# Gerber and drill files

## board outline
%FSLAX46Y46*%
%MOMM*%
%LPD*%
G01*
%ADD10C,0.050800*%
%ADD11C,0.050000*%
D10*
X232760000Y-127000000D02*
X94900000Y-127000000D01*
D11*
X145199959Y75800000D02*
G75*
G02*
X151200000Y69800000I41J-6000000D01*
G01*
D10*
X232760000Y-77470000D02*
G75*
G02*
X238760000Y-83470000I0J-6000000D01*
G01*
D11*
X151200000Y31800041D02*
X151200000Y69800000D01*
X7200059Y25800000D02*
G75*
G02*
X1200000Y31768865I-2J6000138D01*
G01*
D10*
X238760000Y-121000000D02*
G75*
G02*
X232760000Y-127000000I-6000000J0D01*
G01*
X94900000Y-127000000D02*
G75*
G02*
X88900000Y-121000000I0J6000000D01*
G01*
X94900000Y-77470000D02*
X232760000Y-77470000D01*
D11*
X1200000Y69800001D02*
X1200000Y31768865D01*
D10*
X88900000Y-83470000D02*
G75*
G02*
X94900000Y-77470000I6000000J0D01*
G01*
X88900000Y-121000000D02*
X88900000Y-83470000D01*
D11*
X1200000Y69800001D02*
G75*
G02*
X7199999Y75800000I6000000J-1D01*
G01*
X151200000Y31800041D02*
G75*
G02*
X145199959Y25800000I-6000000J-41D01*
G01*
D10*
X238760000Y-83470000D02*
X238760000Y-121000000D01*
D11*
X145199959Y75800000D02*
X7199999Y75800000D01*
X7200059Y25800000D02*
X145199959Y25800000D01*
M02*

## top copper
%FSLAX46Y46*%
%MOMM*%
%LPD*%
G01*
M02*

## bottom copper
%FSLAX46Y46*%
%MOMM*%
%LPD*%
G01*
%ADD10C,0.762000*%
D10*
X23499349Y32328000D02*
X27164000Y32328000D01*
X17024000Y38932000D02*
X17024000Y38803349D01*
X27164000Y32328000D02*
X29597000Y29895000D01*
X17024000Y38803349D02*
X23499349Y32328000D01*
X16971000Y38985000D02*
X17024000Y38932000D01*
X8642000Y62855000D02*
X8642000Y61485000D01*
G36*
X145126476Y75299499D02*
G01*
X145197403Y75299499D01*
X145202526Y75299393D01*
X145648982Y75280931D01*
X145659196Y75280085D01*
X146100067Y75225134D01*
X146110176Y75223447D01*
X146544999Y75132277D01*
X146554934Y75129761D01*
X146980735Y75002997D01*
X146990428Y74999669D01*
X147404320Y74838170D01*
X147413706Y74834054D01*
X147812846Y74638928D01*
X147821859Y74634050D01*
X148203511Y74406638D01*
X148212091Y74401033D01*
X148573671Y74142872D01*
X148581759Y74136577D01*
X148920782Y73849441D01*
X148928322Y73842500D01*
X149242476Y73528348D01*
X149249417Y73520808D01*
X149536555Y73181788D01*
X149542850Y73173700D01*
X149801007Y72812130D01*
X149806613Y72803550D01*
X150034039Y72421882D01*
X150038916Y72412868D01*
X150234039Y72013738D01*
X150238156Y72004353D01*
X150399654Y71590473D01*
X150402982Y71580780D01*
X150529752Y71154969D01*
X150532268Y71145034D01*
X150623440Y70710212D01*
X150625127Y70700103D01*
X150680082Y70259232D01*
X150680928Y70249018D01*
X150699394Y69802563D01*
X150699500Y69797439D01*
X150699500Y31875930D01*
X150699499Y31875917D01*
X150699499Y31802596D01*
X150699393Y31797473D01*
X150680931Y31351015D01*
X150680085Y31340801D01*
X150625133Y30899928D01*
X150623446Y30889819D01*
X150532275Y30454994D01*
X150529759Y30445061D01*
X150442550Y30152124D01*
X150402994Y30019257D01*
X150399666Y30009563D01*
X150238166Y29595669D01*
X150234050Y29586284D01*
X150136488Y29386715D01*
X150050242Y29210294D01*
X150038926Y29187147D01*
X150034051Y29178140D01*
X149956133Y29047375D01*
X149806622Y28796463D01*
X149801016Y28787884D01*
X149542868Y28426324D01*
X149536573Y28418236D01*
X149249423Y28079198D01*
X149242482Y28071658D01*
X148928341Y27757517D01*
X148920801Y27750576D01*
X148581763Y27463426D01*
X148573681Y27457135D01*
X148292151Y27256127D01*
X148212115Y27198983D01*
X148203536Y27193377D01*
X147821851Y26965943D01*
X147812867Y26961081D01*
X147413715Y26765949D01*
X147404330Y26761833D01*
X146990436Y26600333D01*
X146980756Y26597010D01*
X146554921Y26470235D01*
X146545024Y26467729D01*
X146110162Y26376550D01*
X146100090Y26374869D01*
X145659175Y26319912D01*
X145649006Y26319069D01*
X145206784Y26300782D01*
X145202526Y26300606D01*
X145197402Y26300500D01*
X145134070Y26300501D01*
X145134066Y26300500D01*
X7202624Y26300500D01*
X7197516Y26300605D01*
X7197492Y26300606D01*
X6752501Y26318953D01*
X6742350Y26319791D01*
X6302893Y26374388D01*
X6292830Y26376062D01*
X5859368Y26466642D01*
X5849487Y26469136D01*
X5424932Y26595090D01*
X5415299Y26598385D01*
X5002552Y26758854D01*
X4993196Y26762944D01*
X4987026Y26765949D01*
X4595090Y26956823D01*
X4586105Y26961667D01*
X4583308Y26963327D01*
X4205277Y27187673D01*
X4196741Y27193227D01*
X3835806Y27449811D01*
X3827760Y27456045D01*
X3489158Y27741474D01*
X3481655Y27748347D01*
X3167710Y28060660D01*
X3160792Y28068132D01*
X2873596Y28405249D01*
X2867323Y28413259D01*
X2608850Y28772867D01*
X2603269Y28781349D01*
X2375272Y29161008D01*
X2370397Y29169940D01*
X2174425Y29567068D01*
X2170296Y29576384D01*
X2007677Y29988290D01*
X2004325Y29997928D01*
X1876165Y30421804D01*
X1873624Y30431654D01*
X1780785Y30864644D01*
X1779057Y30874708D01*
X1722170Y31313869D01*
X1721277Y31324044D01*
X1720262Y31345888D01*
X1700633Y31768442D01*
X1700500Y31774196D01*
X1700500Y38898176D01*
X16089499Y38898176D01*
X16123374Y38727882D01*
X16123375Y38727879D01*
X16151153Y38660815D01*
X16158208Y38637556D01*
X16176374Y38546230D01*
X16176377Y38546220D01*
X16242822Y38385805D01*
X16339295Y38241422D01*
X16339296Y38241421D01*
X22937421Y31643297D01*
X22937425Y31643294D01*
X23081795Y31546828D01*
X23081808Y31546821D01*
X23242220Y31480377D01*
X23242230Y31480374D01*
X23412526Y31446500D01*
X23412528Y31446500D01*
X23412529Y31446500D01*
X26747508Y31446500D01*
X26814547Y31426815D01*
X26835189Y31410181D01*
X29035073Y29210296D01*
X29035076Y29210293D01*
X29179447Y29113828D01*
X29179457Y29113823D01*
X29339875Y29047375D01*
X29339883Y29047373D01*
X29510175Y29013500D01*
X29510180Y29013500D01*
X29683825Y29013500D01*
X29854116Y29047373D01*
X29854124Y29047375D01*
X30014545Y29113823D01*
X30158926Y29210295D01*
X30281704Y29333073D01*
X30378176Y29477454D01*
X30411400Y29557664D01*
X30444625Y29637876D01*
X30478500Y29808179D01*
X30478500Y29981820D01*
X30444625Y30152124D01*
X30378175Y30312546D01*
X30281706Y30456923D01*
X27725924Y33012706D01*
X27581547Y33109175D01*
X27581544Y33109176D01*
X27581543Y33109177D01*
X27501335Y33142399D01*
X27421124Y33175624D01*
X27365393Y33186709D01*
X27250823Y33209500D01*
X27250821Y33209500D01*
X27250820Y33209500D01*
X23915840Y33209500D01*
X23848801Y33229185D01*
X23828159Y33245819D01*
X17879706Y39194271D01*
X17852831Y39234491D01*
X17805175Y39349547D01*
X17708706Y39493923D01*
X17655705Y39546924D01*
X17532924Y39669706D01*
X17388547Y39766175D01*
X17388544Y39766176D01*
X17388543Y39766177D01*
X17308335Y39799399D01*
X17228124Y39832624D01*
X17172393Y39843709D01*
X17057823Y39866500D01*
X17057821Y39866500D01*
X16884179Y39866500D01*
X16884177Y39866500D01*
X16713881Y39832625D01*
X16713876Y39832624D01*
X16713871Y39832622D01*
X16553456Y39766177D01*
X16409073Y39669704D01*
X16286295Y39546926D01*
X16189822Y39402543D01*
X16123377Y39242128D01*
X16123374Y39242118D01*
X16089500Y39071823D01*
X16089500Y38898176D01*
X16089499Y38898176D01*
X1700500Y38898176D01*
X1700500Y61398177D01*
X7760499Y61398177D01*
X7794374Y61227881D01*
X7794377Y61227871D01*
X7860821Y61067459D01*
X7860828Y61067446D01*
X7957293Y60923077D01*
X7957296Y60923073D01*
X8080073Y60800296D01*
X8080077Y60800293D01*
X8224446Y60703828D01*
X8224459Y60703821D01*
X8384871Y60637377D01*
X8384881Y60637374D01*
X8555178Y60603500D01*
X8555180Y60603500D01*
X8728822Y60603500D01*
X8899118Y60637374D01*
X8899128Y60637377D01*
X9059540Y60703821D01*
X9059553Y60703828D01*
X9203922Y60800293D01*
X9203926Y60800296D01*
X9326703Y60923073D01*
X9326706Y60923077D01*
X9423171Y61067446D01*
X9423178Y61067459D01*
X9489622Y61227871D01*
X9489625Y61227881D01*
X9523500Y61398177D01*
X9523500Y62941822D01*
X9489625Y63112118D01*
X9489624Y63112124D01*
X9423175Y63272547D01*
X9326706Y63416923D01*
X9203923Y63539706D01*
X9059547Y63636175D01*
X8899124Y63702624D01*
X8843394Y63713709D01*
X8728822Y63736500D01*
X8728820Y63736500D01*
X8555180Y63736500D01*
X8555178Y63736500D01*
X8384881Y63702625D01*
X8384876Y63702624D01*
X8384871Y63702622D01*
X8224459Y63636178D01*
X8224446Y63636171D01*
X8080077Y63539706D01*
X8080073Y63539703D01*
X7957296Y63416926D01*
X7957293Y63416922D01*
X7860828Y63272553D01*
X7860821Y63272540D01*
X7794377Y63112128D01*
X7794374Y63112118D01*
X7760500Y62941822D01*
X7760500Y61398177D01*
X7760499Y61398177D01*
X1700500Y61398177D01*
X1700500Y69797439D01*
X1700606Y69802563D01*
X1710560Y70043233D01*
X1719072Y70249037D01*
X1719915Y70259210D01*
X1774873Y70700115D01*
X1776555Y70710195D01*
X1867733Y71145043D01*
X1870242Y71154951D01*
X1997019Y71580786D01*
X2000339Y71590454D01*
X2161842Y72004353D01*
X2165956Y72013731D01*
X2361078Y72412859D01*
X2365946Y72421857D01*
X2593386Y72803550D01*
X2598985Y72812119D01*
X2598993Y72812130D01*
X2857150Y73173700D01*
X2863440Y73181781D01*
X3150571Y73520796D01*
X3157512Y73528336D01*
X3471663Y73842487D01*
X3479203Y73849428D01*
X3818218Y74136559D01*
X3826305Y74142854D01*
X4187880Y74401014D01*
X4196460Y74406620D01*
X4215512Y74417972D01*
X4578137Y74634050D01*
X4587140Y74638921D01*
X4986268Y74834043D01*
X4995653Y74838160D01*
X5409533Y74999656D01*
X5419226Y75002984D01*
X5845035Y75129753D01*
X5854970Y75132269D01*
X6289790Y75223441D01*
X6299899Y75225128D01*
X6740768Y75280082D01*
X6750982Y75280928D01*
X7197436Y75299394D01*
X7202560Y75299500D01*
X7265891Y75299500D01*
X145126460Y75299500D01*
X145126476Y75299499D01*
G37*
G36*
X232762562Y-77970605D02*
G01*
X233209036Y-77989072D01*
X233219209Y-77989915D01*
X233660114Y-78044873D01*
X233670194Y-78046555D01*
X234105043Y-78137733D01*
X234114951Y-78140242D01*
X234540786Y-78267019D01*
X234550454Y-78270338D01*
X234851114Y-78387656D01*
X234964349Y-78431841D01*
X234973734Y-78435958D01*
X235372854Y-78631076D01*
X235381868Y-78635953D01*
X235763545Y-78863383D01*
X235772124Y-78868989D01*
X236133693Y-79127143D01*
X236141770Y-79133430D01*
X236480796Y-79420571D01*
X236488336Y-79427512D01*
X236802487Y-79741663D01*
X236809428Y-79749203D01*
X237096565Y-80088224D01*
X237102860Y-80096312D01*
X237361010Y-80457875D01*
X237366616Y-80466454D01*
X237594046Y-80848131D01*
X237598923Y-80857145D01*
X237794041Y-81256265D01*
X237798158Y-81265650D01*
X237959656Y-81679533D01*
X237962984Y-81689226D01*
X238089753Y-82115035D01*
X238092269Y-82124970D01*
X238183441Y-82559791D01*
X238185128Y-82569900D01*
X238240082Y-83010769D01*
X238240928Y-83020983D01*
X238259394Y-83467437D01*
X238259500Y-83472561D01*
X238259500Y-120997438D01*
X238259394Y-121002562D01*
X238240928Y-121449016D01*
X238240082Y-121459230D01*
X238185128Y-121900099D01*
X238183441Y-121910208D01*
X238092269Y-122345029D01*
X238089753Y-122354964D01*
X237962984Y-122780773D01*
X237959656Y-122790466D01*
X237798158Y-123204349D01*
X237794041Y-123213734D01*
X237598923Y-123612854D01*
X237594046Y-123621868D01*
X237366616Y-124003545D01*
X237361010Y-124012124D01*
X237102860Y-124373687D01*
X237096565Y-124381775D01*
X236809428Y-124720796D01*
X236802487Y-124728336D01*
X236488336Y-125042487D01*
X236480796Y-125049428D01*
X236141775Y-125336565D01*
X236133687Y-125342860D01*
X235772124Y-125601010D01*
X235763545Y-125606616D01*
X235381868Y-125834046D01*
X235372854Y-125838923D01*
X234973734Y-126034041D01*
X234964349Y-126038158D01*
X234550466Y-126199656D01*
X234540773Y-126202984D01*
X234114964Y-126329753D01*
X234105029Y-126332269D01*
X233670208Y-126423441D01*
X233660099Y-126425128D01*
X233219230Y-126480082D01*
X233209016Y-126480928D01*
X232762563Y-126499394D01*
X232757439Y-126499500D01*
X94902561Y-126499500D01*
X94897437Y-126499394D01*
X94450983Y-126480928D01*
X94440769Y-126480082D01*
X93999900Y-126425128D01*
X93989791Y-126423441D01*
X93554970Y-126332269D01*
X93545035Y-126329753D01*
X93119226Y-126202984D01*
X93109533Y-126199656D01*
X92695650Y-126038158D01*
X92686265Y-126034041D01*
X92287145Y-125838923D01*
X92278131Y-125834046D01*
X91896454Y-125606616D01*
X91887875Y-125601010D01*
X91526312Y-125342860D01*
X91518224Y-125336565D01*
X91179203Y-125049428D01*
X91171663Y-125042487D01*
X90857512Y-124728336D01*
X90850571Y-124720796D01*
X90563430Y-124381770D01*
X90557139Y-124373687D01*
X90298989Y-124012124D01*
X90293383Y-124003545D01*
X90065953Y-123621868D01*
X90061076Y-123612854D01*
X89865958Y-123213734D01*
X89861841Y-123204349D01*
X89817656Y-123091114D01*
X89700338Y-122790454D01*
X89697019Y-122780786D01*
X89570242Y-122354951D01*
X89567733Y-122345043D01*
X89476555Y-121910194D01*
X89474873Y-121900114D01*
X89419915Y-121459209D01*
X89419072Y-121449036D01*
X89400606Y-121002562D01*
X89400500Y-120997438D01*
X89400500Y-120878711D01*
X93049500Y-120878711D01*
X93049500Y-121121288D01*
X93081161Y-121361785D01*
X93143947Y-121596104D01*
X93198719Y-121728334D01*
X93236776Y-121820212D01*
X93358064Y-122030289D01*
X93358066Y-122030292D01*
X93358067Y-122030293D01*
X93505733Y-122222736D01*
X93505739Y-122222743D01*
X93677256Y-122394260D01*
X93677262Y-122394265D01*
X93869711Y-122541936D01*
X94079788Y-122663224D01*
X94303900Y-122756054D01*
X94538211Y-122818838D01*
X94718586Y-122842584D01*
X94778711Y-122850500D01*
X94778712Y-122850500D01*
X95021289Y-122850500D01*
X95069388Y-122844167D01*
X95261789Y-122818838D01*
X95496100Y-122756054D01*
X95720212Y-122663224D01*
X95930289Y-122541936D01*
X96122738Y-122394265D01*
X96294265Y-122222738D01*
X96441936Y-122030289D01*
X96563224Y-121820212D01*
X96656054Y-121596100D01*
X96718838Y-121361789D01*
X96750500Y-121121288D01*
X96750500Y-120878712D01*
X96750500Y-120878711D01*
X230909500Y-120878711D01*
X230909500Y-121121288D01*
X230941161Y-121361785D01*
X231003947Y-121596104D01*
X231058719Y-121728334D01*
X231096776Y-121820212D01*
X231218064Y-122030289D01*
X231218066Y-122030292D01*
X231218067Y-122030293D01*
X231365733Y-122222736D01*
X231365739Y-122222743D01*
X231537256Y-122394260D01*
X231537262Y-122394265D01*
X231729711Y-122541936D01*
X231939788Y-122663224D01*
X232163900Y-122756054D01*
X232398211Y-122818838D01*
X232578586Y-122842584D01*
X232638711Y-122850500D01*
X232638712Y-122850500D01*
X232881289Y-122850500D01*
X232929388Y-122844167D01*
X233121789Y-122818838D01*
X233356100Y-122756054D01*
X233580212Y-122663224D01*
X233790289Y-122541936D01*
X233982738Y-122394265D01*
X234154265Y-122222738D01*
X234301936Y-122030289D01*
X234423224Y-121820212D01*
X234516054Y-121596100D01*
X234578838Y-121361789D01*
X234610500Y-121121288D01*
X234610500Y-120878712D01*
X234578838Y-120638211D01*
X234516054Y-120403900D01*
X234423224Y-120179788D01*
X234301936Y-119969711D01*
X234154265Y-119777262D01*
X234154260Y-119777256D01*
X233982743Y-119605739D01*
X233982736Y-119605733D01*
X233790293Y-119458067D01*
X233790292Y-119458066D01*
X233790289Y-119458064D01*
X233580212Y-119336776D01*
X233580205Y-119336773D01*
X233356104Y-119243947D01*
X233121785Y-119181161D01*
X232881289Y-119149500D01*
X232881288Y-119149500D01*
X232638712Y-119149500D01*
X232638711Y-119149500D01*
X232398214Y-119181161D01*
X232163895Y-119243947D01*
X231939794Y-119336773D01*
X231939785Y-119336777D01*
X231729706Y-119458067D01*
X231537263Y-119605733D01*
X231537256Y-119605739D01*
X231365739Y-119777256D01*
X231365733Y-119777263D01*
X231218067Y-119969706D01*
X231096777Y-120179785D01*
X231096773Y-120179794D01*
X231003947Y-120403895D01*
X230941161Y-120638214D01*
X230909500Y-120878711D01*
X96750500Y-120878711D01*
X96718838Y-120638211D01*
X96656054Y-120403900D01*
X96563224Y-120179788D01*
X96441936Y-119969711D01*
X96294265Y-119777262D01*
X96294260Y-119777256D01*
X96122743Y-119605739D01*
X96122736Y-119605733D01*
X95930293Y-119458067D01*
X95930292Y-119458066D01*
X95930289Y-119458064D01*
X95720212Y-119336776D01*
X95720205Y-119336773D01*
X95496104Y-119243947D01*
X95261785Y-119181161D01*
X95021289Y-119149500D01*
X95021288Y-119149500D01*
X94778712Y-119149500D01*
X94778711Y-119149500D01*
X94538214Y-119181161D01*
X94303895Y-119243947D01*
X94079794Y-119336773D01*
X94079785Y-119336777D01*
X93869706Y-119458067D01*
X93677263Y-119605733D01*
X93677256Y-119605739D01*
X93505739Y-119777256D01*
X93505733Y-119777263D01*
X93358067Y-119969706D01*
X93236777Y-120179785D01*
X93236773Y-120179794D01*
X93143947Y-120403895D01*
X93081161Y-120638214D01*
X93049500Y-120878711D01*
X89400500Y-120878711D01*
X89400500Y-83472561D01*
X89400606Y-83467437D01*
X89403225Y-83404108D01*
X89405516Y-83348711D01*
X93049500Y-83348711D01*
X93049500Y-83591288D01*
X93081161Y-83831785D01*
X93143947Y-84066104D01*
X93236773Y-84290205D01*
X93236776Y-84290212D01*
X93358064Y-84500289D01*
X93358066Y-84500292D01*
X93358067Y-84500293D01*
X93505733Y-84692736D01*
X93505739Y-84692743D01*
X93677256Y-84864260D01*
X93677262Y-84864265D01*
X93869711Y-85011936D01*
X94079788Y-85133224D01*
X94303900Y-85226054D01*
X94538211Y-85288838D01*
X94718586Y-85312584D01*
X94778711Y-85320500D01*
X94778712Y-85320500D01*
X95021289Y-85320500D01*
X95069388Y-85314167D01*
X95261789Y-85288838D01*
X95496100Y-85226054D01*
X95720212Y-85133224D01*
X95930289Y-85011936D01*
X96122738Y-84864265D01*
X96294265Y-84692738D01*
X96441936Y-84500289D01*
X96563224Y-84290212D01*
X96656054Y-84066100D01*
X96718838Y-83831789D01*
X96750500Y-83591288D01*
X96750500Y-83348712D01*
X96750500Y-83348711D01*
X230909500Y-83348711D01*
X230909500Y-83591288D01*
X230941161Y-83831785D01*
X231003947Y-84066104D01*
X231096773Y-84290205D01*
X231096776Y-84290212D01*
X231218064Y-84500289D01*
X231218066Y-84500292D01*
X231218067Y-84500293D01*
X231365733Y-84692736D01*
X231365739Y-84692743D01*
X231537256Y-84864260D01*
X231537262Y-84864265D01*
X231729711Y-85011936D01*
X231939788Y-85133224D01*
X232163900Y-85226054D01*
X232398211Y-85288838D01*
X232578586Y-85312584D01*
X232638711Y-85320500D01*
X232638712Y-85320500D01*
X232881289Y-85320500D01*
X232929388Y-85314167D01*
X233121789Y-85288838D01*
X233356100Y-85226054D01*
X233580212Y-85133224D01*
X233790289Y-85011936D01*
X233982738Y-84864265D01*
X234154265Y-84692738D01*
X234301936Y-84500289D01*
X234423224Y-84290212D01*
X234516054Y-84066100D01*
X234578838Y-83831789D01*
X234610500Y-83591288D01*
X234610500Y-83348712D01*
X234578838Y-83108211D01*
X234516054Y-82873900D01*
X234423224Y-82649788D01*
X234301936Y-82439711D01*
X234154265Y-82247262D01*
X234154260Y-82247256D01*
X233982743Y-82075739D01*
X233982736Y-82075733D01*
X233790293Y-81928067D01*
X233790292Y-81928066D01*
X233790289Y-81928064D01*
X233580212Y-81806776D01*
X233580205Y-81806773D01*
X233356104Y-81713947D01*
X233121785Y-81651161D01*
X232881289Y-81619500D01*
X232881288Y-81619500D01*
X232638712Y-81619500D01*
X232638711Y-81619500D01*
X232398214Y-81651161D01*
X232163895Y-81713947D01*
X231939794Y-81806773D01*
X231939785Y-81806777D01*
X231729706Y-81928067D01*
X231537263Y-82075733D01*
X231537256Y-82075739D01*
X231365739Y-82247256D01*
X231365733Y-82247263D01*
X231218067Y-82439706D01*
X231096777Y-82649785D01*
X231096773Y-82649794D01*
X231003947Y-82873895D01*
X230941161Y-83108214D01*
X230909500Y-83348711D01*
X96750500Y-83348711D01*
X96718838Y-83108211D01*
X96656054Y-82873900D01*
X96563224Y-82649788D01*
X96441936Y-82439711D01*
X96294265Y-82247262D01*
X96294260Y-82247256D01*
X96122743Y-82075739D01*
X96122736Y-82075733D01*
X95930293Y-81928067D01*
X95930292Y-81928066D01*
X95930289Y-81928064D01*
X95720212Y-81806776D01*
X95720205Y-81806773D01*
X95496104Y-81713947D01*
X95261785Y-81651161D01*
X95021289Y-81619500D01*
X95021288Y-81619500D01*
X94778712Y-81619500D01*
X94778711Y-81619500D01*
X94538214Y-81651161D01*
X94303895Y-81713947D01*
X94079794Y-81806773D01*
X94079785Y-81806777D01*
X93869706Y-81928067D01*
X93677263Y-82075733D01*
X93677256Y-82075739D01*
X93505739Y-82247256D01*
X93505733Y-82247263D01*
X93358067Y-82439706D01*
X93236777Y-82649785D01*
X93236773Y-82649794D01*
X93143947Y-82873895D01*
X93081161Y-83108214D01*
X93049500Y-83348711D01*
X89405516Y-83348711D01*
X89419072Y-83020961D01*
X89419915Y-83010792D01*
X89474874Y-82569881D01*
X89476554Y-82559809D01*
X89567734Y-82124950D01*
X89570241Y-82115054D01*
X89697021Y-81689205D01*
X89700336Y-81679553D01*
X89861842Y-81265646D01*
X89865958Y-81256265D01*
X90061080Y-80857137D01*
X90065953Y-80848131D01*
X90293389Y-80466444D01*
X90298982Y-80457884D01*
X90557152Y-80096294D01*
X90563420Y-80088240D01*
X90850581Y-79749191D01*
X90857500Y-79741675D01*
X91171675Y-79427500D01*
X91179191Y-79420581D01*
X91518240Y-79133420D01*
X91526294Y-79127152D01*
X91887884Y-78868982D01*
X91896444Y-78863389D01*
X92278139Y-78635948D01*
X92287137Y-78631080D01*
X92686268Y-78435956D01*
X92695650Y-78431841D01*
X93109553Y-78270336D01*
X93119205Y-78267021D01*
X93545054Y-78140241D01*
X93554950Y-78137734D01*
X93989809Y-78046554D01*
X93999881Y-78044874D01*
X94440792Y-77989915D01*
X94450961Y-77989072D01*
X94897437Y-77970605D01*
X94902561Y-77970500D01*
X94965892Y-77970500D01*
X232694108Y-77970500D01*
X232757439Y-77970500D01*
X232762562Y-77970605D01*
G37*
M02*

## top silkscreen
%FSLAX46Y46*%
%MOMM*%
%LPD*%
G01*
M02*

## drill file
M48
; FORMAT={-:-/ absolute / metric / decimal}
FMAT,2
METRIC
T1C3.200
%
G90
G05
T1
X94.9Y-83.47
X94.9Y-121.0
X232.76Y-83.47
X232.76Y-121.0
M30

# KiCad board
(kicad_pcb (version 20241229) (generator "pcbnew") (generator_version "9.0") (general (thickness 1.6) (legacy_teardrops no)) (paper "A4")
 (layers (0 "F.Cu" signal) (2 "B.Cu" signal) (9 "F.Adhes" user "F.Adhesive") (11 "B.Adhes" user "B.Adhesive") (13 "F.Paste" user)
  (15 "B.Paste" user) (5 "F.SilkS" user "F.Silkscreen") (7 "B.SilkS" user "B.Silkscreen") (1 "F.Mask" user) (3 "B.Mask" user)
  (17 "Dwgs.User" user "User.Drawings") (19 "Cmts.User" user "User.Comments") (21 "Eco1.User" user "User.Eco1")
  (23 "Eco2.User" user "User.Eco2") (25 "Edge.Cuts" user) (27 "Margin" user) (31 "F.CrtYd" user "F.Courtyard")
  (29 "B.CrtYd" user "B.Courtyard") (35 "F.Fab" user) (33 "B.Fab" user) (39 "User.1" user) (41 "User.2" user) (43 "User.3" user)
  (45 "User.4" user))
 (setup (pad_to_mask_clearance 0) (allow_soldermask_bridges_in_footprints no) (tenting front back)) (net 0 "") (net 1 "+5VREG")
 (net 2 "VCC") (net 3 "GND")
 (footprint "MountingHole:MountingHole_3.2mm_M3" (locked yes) (layer "F.Cu") (at 232.76 121)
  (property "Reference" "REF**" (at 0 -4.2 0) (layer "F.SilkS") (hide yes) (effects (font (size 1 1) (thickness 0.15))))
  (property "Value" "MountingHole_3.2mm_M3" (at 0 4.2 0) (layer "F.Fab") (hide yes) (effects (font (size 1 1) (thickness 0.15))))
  (pad "" np_thru_hole circle (at 0 0) (size 3.2 3.2) (drill 3.2) (layers "*.Cu" "*.Mask")))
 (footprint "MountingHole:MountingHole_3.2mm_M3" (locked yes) (layer "F.Cu") (at 94.9 83.47)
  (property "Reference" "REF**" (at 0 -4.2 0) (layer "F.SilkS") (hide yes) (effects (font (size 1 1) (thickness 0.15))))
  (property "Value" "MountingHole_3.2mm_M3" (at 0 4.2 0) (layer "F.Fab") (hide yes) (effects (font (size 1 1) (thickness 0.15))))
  (pad "" np_thru_hole circle (at 0 0) (size 3.2 3.2) (drill 3.2) (layers "*.Cu" "*.Mask")))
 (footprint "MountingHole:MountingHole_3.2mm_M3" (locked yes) (layer "F.Cu") (at 94.9 121)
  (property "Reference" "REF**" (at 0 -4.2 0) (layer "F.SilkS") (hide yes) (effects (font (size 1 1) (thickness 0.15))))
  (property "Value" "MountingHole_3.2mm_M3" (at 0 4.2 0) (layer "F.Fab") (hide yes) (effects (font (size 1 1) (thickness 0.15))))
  (pad "" np_thru_hole circle (at 0 0) (size 3.2 3.2) (drill 3.2) (layers "*.Cu" "*.Mask")))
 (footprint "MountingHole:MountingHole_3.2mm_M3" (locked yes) (layer "F.Cu") (at 232.76 83.47)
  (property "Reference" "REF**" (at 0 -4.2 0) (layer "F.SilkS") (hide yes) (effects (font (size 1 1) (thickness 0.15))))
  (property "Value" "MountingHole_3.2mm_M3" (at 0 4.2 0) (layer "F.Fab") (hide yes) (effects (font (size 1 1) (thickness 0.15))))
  (pad "" np_thru_hole circle (at 0 0) (size 3.2 3.2) (drill 3.2) (layers "*.Cu" "*.Mask")))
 (gr_line (start 232.76 127) (end 94.9 127) (stroke (width 0.0508) (type default)) (layer "Edge.Cuts"))
 (gr_arc (start 145.199959 -75.8) (mid 149.442641 -74.042641) (end 151.2 -69.8) (stroke (width 0.05) (type default)) (layer "Edge.Cuts"))
 (gr_arc (start 232.76 77.47) (mid 237.002641 79.227359) (end 238.76 83.47) (stroke (width 0.0508) (type default)) (layer "Edge.Cuts"))
 (gr_line (start 151.2 -31.800041) (end 151.2 -69.8) (stroke (width 0.05) (type default)) (layer "Edge.Cuts"))
 (gr_arc (start 7.200059 -25.8) (mid 2.957359 -27.557359) (end 1.2 -31.768865) (stroke (width 0.05) (type default)) (layer "Edge.Cuts"))
 (gr_arc (start 238.76 121) (mid 237.002641 125.242641) (end 232.76 127) (stroke (width 0.0508) (type default)) (layer "Edge.Cuts"))
 (gr_arc (start 94.9 127) (mid 90.657359 125.242641) (end 88.9 121) (stroke (width 0.0508) (type default)) (layer "Edge.Cuts"))
 (gr_line (start 94.9 77.47) (end 232.76 77.47) (stroke (width 0.0508) (type default)) (layer "Edge.Cuts"))
 (gr_line (start 1.2 -69.800001) (end 1.2 -31.768865) (stroke (width 0.05) (type default)) (layer "Edge.Cuts"))
 (gr_arc (start 88.9 83.47) (mid 90.657359 79.227359) (end 94.9 77.47) (stroke (width 0.0508) (type default)) (layer "Edge.Cuts"))
 (gr_line (start 88.9 121) (end 88.9 83.47) (stroke (width 0.0508) (type default)) (layer "Edge.Cuts"))
 (gr_arc (start 1.2 -69.800001) (mid 2.957359 -74.042641) (end 7.199999 -75.8) (stroke (width 0.05) (type default)) (layer "Edge.Cuts"))
 (gr_arc (start 151.2 -31.800041) (mid 149.442641 -27.557359) (end 145.199959 -25.8) (stroke (width 0.05) (type default))
  (layer "Edge.Cuts"))
 (gr_line (start 238.76 83.47) (end 238.76 121) (stroke (width 0.0508) (type default)) (layer "Edge.Cuts"))
 (gr_line (start 145.199959 -75.8) (end 7.199999 -75.8) (stroke (width 0.05) (type default)) (layer "Edge.Cuts"))
 (gr_line (start 7.200059 -25.8) (end 145.199959 -25.8) (stroke (width 0.05) (type default)) (layer "Edge.Cuts"))
 (segment (start 23.499349 -32.328) (end 27.164 -32.328) (width 0.762) (layer "B.Cu") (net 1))
 (segment (start 17.024 -38.932) (end 17.024 -38.803349) (width 0.762) (layer "B.Cu") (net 1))
 (segment (start 27.164 -32.328) (end 29.597 -29.895) (width 0.762) (layer "B.Cu") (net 1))
 (segment (start 17.024 -38.803349) (end 23.499349 -32.328) (width 0.762) (layer "B.Cu") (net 1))
 (segment (start 16.971 -38.985) (end 17.024 -38.932) (width 0.762) (layer "B.Cu") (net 1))
 (segment (start 8.642 -62.855) (end 8.642 -61.485) (width 0.762) (layer "B.Cu") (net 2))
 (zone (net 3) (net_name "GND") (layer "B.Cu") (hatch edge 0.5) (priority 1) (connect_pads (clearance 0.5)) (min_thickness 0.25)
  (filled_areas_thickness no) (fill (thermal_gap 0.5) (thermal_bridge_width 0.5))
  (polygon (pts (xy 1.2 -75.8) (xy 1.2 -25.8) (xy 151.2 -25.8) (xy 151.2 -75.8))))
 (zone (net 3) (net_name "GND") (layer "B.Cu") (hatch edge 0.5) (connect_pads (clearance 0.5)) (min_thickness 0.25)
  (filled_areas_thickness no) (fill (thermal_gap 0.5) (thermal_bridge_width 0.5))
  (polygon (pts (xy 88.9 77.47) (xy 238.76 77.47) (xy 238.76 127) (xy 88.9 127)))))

